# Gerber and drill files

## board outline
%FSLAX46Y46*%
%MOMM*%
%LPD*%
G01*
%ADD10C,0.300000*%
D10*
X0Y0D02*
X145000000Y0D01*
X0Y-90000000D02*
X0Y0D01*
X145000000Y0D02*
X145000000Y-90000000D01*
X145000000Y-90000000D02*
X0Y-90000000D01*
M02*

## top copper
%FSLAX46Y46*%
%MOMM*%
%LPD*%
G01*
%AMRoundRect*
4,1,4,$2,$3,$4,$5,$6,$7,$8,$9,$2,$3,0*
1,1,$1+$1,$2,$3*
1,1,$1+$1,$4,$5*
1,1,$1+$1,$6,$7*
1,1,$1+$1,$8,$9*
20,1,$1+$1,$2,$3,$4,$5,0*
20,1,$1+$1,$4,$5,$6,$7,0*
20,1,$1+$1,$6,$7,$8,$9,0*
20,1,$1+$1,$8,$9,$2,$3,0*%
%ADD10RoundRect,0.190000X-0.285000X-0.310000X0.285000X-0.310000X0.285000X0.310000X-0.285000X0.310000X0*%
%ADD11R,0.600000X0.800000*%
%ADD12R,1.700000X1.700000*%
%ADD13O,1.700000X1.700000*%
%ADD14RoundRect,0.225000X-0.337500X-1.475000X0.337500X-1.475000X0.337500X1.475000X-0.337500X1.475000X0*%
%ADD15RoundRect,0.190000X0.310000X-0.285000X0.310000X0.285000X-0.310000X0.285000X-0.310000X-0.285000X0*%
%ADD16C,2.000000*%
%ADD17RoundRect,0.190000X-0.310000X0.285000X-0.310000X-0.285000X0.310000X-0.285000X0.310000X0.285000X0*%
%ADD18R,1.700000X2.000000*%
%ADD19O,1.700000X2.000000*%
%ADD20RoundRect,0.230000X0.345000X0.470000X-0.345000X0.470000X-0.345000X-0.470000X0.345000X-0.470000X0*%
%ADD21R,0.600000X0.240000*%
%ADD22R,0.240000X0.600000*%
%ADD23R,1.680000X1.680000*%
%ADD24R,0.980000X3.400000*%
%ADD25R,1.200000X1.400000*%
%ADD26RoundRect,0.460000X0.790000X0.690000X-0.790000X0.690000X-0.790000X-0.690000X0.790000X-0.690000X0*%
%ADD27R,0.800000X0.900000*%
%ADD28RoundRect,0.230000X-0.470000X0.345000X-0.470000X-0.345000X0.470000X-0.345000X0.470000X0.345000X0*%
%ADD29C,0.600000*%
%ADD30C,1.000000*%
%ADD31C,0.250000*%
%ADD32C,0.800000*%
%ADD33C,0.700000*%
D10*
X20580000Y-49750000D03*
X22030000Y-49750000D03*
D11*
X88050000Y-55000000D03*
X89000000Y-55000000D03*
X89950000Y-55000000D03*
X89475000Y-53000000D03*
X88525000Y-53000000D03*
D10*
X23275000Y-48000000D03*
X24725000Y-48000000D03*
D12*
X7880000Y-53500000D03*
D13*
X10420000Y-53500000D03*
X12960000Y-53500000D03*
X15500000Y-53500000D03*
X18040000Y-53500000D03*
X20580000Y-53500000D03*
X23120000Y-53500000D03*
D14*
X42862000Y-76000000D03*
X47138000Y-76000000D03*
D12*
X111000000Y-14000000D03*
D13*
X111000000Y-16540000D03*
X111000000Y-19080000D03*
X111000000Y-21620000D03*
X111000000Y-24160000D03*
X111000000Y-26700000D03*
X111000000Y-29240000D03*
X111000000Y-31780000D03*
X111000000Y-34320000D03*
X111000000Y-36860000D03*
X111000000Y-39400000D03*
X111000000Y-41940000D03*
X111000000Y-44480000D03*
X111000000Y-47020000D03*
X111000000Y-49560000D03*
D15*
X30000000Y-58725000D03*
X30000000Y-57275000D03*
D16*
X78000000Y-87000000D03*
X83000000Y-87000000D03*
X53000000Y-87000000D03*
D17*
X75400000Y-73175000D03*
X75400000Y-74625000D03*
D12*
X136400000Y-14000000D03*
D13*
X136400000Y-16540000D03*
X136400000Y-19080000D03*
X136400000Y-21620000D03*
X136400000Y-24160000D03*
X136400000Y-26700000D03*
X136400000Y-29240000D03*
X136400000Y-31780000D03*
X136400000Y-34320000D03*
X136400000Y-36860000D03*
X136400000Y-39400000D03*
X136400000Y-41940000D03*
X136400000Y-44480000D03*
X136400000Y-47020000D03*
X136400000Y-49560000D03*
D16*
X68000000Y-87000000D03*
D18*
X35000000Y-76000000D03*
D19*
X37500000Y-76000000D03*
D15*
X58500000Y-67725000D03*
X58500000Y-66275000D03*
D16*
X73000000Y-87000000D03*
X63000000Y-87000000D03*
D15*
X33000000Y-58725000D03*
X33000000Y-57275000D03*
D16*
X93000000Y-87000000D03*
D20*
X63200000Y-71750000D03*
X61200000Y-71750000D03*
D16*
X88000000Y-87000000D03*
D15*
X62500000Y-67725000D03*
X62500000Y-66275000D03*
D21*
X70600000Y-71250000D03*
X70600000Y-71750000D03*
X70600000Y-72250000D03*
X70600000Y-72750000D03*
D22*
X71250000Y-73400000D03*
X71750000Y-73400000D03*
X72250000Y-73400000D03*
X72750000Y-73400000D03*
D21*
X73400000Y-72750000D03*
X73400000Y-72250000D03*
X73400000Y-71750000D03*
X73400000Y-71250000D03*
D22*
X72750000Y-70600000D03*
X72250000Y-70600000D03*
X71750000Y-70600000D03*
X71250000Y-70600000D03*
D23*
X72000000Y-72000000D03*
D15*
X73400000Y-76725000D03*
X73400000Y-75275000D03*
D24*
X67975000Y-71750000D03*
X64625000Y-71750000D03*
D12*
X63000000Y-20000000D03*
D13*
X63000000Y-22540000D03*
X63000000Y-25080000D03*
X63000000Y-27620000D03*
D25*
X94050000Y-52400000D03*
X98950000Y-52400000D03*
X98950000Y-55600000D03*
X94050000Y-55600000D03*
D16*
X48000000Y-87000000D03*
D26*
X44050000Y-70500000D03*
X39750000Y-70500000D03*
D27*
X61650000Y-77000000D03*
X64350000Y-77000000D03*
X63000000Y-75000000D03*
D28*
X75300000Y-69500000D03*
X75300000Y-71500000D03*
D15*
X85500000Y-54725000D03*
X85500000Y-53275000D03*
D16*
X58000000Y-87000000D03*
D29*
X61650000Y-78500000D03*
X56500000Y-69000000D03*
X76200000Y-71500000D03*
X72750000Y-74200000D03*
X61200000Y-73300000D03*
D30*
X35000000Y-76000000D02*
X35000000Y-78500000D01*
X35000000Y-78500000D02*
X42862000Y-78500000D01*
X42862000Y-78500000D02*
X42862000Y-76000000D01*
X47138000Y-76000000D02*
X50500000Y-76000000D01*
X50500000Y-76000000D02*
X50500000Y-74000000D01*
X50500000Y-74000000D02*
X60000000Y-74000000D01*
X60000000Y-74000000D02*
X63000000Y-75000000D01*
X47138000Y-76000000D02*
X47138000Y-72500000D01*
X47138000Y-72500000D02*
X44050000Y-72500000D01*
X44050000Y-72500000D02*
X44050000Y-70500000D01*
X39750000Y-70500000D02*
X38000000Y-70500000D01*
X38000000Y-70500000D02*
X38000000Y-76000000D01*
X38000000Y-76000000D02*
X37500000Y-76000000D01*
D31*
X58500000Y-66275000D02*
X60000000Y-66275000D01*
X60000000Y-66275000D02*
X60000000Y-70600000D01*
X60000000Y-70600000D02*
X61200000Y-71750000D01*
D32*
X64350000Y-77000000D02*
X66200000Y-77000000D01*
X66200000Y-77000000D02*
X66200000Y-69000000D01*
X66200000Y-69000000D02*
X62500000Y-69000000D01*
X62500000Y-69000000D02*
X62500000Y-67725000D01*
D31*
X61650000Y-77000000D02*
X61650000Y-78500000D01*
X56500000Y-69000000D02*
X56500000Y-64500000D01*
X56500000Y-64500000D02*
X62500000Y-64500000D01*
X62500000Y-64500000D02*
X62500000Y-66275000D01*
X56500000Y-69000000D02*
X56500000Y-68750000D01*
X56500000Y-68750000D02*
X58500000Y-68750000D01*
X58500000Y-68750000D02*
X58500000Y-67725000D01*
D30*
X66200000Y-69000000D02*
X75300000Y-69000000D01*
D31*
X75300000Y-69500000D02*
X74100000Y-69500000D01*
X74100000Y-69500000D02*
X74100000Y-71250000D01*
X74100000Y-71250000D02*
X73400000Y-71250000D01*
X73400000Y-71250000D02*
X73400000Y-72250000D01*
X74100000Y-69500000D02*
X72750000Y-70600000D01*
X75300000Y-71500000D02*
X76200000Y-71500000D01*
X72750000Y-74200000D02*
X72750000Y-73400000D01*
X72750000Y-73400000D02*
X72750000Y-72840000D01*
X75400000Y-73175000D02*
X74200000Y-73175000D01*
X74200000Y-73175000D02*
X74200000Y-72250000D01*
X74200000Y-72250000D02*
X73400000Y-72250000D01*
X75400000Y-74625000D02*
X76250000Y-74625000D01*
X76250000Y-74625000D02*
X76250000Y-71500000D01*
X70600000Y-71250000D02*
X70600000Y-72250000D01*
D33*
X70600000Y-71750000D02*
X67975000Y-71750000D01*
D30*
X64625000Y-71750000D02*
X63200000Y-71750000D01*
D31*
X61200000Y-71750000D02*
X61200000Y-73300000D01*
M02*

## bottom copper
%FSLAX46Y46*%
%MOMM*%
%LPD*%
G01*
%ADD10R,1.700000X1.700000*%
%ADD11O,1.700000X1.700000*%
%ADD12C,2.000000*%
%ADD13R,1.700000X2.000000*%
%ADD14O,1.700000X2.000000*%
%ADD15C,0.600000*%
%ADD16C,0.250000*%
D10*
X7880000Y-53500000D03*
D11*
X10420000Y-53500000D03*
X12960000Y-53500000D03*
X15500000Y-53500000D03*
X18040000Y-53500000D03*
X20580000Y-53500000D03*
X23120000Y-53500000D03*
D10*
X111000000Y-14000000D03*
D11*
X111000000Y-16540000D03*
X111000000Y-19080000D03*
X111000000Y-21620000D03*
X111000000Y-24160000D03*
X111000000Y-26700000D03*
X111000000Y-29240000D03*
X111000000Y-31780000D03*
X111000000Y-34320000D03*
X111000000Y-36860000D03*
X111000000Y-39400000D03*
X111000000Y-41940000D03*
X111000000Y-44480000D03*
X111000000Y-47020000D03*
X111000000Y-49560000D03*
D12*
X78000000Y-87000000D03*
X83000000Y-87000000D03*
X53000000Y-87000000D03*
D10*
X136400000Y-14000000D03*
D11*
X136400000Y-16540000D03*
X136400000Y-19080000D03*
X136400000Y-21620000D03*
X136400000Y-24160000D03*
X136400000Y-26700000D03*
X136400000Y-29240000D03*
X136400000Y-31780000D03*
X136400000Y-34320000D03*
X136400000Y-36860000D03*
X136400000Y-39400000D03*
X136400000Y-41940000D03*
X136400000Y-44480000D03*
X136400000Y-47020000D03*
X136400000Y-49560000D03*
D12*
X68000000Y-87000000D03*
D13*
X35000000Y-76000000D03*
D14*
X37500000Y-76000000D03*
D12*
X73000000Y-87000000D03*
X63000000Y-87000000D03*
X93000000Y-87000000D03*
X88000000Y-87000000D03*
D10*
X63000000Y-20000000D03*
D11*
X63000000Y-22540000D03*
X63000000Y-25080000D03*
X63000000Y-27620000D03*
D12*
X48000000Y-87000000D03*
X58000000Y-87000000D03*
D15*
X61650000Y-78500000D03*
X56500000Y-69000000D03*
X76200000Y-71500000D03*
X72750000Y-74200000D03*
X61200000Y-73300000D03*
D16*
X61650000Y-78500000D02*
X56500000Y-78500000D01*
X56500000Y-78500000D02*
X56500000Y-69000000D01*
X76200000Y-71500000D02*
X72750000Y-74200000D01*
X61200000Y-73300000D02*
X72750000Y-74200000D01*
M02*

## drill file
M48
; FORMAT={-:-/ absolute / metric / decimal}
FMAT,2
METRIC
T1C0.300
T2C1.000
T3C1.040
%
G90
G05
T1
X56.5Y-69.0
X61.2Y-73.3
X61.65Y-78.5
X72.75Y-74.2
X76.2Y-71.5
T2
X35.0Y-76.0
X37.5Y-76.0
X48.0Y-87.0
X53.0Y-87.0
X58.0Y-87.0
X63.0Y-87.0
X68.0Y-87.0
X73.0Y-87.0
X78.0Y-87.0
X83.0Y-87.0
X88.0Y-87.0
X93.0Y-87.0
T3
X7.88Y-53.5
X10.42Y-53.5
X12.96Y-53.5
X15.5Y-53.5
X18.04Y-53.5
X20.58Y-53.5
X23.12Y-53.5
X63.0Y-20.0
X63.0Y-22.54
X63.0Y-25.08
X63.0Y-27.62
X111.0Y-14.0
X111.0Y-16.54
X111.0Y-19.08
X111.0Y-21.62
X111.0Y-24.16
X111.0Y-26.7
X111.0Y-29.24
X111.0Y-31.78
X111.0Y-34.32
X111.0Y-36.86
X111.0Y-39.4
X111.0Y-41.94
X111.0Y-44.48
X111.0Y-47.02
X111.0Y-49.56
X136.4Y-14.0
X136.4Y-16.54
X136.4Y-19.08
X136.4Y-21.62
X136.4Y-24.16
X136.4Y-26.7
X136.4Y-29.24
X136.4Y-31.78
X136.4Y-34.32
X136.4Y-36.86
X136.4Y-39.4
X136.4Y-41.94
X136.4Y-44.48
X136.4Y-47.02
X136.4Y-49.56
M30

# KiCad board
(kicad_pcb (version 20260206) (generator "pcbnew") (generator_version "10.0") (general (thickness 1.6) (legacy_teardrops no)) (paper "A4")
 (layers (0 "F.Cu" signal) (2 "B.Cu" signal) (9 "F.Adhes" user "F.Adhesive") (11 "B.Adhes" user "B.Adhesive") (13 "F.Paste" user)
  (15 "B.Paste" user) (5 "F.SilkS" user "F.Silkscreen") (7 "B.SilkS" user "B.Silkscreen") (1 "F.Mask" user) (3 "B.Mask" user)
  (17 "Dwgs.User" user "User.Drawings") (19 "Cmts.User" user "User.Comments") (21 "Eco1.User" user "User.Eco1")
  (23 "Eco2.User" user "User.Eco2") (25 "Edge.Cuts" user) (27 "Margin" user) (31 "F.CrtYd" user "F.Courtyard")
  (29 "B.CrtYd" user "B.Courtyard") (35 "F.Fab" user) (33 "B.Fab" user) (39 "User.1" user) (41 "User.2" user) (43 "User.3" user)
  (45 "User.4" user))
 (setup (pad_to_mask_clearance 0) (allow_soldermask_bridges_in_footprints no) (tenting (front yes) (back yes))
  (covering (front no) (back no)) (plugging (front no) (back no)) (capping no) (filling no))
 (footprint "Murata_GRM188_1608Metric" (layer "F.Cu") (at 21.305 49.75)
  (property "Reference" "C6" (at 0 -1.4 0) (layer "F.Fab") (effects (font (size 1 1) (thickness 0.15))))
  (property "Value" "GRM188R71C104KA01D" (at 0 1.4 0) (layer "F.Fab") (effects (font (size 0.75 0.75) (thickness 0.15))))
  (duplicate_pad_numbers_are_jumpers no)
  (pad "1" smd roundrect (at -0.725 0) (size 0.95 1) (layers "F.Cu" "F.Mask" "F.Paste") (roundrect_rratio 0.2) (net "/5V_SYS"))
  (pad "2" smd roundrect (at 0.725 0) (size 0.95 1) (layers "F.Cu" "F.Mask" "F.Paste") (roundrect_rratio 0.2) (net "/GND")))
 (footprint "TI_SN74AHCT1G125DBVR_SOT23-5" (layer "F.Cu") (at 89 54)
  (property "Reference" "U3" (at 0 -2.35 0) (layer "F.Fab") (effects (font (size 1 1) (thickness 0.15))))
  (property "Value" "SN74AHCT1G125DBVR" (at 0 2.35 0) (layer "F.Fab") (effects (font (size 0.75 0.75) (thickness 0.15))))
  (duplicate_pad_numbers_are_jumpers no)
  (pad "1" smd rect (at -0.95 1) (size 0.6 0.8) (layers "F.Cu" "F.Mask" "F.Paste") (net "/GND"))
  (pad "2" smd rect (at 0 1) (size 0.6 0.8) (layers "F.Cu" "F.Mask" "F.Paste") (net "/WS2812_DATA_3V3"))
  (pad "3" smd rect (at 0.95 1) (size 0.6 0.8) (layers "F.Cu" "F.Mask" "F.Paste") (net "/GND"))
  (pad "4" smd rect (at 0.475 -1) (size 0.6 0.8) (layers "F.Cu" "F.Mask" "F.Paste") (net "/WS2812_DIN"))
  (pad "5" smd rect (at -0.475 -1) (size 0.6 0.8) (layers "F.Cu" "F.Mask" "F.Paste") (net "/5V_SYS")))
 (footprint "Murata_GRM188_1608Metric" (layer "F.Cu") (at 24 48)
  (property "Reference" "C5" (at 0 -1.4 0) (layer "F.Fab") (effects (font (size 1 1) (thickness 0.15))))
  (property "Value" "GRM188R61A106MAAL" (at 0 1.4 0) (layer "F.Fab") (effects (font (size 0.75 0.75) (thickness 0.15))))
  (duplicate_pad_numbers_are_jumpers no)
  (pad "1" smd roundrect (at -0.725 0) (size 0.95 1) (layers "F.Cu" "F.Mask" "F.Paste") (roundrect_rratio 0.2) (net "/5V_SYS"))
  (pad "2" smd roundrect (at 0.725 0) (size 0.95 1) (layers "F.Cu" "F.Mask" "F.Paste") (roundrect_rratio 0.2) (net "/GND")))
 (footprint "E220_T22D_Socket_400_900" (layer "F.Cu") (at 5 52)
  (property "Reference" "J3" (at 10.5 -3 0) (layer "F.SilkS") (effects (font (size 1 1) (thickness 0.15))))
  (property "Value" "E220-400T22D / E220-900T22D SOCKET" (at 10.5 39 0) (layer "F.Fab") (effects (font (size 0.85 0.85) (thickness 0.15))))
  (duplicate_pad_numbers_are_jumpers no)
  (pad "1" thru_hole rect (at 2.88 1.5) (size 1.7 1.7) (drill 1.04) (layers "*.Cu" "*.Mask") (remove_unused_layers no) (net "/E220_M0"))
  (pad "2" thru_hole oval (at 5.42 1.5) (size 1.7 1.7) (drill 1.04) (layers "*.Cu" "*.Mask") (remove_unused_layers no) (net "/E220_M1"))
  (pad "3" thru_hole oval (at 7.96 1.5) (size 1.7 1.7) (drill 1.04) (layers "*.Cu" "*.Mask") (remove_unused_layers no) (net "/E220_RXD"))
  (pad "4" thru_hole oval (at 10.5 1.5) (size 1.7 1.7) (drill 1.04) (layers "*.Cu" "*.Mask") (remove_unused_layers no) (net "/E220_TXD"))
  (pad "5" thru_hole oval (at 13.04 1.5) (size 1.7 1.7) (drill 1.04) (layers "*.Cu" "*.Mask") (remove_unused_layers no) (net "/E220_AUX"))
  (pad "6" thru_hole oval (at 15.58 1.5) (size 1.7 1.7) (drill 1.04) (layers "*.Cu" "*.Mask") (remove_unused_layers no) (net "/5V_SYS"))
  (pad "7" thru_hole oval (at 18.12 1.5) (size 1.7 1.7) (drill 1.04) (layers "*.Cu" "*.Mask") (remove_unused_layers no) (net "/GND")))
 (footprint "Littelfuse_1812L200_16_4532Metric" (layer "F.Cu") (at 45 76)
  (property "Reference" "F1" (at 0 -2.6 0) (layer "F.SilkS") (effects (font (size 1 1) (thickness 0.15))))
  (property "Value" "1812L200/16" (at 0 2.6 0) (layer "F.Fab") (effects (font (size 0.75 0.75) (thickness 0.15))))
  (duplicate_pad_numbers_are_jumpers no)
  (pad "1" smd roundrect (at -2.138 0) (size 1.125 3.4) (layers "F.Cu" "F.Mask" "F.Paste") (roundrect_rratio 0.2) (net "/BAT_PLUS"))
  (pad "2" smd roundrect (at 2.138 0) (size 1.125 3.4) (layers "F.Cu" "F.Mask" "F.Paste") (roundrect_rratio 0.2) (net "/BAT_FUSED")))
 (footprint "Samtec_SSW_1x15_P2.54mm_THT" (layer "F.Cu") (at 111 14)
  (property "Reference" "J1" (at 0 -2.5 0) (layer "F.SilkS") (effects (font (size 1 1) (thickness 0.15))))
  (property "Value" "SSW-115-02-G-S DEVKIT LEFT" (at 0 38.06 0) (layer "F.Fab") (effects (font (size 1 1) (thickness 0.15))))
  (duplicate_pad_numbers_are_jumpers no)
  (pad "1" thru_hole rect (at 0 0) (size 1.7 1.7) (drill 1.04) (layers "*.Cu" "*.Mask") (remove_unused_layers no) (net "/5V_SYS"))
  (pad "2" thru_hole oval (at 0 2.54) (size 1.7 1.7) (drill 1.04) (layers "*.Cu" "*.Mask") (remove_unused_layers no) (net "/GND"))
  (pad "3" thru_hole oval (at 0 5.08) (size 1.7 1.7) (drill 1.04) (layers "*.Cu" "*.Mask") (remove_unused_layers no))
  (pad "4" thru_hole oval (at 0 7.62) (size 1.7 1.7) (drill 1.04) (layers "*.Cu" "*.Mask") (remove_unused_layers no))
  (pad "5" thru_hole oval (at 0 10.16) (size 1.7 1.7) (drill 1.04) (layers "*.Cu" "*.Mask") (remove_unused_layers no))
  (pad "6" thru_hole oval (at 0 12.7) (size 1.7 1.7) (drill 1.04) (layers "*.Cu" "*.Mask") (remove_unused_layers no) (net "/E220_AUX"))
  (pad "7" thru_hole oval (at 0 15.24) (size 1.7 1.7) (drill 1.04) (layers "*.Cu" "*.Mask") (remove_unused_layers no) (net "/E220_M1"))
  (pad "8" thru_hole oval (at 0 17.78) (size 1.7 1.7) (drill 1.04) (layers "*.Cu" "*.Mask") (remove_unused_layers no) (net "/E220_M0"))
  (pad "9" thru_hole oval (at 0 20.32) (size 1.7 1.7) (drill 1.04) (layers "*.Cu" "*.Mask") (remove_unused_layers no))
  (pad "10" thru_hole oval (at 0 22.86) (size 1.7 1.7) (drill 1.04) (layers "*.Cu" "*.Mask") (remove_unused_layers no))
  (pad "11" thru_hole oval (at 0 25.4) (size 1.7 1.7) (drill 1.04) (layers "*.Cu" "*.Mask") (remove_unused_layers no))
  (pad "12" thru_hole oval (at 0 27.94) (size 1.7 1.7) (drill 1.04) (layers "*.Cu" "*.Mask") (remove_unused_layers no))
  (pad "13" thru_hole oval (at 0 30.48) (size 1.7 1.7) (drill 1.04) (layers "*.Cu" "*.Mask") (remove_unused_layers no))
  (pad "14" thru_hole oval (at 0 33.02) (size 1.7 1.7) (drill 1.04) (layers "*.Cu" "*.Mask") (remove_unused_layers no))
  (pad "15" thru_hole oval (at 0 35.56) (size 1.7 1.7) (drill 1.04) (layers "*.Cu" "*.Mask") (remove_unused_layers no)))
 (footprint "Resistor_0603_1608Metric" (layer "F.Cu") (at 30 58 90)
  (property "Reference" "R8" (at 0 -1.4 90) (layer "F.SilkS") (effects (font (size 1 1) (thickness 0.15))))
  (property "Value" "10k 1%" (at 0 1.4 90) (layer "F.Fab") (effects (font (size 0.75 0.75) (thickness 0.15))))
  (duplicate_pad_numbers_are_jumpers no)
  (pad "1" smd roundrect (at -0.725 0 90) (size 0.95 1) (layers "F.Cu" "F.Mask" "F.Paste") (roundrect_rratio 0.2) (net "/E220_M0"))
  (pad "2" smd roundrect (at 0.725 0 90) (size 0.95 1) (layers "F.Cu" "F.Mask" "F.Paste") (roundrect_rratio 0.2) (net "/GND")))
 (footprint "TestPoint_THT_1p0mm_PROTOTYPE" (layer "F.Cu") (at 78 87)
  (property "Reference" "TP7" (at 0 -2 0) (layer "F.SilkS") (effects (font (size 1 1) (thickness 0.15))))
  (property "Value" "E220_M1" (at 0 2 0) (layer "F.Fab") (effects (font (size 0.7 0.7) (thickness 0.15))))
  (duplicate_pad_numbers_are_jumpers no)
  (pad "1" thru_hole circle (at 0 0) (size 2 2) (drill 1) (layers "*.Cu" "*.Mask") (remove_unused_layers no) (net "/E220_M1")))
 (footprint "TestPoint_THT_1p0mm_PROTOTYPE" (layer "F.Cu") (at 83 87)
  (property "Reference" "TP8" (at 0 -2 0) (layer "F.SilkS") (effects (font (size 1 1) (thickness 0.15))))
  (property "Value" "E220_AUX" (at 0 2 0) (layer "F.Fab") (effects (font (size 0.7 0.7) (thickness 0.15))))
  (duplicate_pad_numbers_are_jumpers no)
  (pad "1" thru_hole circle (at 0 0) (size 2 2) (drill 1) (layers "*.Cu" "*.Mask") (remove_unused_layers no) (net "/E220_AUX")))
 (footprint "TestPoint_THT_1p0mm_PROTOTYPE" (layer "F.Cu") (at 53 87)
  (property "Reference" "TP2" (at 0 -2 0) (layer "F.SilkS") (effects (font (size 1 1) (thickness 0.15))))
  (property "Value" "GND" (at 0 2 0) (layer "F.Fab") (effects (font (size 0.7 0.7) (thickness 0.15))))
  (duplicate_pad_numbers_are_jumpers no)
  (pad "1" thru_hole circle (at 0 0) (size 2 2) (drill 1) (layers "*.Cu" "*.Mask") (remove_unused_layers no) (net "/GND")))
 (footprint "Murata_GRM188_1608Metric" (layer "F.Cu") (at 75.4 73.9 -90)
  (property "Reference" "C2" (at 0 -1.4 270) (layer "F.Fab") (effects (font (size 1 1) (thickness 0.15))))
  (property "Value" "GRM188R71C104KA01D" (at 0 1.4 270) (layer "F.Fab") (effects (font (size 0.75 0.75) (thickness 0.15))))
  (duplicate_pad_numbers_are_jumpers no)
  (pad "1" smd roundrect (at -0.725 0 270) (size 0.95 1) (layers "F.Cu" "F.Mask" "F.Paste") (roundrect_rratio 0.2) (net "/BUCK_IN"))
  (pad "2" smd roundrect (at 0.725 0 270) (size 0.95 1) (layers "F.Cu" "F.Mask" "F.Paste") (roundrect_rratio 0.2) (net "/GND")))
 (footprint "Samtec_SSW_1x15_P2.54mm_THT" (layer "F.Cu") (at 136.4 14)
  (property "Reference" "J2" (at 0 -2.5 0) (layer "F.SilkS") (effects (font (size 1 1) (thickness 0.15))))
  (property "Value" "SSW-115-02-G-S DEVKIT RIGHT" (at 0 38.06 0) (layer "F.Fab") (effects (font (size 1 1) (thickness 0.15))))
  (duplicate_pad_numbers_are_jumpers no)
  (pad "1" thru_hole rect (at 0 0) (size 1.7 1.7) (drill 1.04) (layers "*.Cu" "*.Mask") (remove_unused_layers no) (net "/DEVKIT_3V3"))
  (pad "2" thru_hole oval (at 0 2.54) (size 1.7 1.7) (drill 1.04) (layers "*.Cu" "*.Mask") (remove_unused_layers no) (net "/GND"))
  (pad "3" thru_hole oval (at 0 5.08) (size 1.7 1.7) (drill 1.04) (layers "*.Cu" "*.Mask") (remove_unused_layers no))
  (pad "4" thru_hole oval (at 0 7.62) (size 1.7 1.7) (drill 1.04) (layers "*.Cu" "*.Mask") (remove_unused_layers no))
  (pad "5" thru_hole oval (at 0 10.16) (size 1.7 1.7) (drill 1.04) (layers "*.Cu" "*.Mask") (remove_unused_layers no)
   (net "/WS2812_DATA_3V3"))
  (pad "6" thru_hole oval (at 0 12.7) (size 1.7 1.7) (drill 1.04) (layers "*.Cu" "*.Mask") (remove_unused_layers no) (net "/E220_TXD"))
  (pad "7" thru_hole oval (at 0 15.24) (size 1.7 1.7) (drill 1.04) (layers "*.Cu" "*.Mask") (remove_unused_layers no) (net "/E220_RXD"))
  (pad "8" thru_hole oval (at 0 17.78) (size 1.7 1.7) (drill 1.04) (layers "*.Cu" "*.Mask") (remove_unused_layers no))
  (pad "9" thru_hole oval (at 0 20.32) (size 1.7 1.7) (drill 1.04) (layers "*.Cu" "*.Mask") (remove_unused_layers no))
  (pad "10" thru_hole oval (at 0 22.86) (size 1.7 1.7) (drill 1.04) (layers "*.Cu" "*.Mask") (remove_unused_layers no))
  (pad "11" thru_hole oval (at 0 25.4) (size 1.7 1.7) (drill 1.04) (layers "*.Cu" "*.Mask") (remove_unused_layers no) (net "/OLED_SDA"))
  (pad "12" thru_hole oval (at 0 27.94) (size 1.7 1.7) (drill 1.04) (layers "*.Cu" "*.Mask") (remove_unused_layers no))
  (pad "13" thru_hole oval (at 0 30.48) (size 1.7 1.7) (drill 1.04) (layers "*.Cu" "*.Mask") (remove_unused_layers no))
  (pad "14" thru_hole oval (at 0 33.02) (size 1.7 1.7) (drill 1.04) (layers "*.Cu" "*.Mask") (remove_unused_layers no) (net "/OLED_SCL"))
  (pad "15" thru_hole oval (at 0 35.56) (size 1.7 1.7) (drill 1.04) (layers "*.Cu" "*.Mask") (remove_unused_layers no)))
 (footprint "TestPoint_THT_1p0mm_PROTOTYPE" (layer "F.Cu") (at 68 87)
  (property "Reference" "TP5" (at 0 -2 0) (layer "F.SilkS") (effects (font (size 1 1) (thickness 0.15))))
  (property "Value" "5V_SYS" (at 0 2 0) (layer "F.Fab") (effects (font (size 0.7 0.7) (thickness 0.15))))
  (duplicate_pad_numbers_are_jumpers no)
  (pad "1" thru_hole circle (at 0 0) (size 2 2) (drill 1) (layers "*.Cu" "*.Mask") (remove_unused_layers no) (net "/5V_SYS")))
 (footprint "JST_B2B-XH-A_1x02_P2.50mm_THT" (layer "F.Cu") (at 35 76)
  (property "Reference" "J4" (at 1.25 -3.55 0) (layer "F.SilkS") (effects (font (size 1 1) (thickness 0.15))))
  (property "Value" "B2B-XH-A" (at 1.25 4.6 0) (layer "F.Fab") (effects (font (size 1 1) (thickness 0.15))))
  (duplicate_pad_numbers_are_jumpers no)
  (pad "1" thru_hole rect (at 0 0) (size 1.7 2) (drill 1) (layers "*.Cu" "*.Mask") (remove_unused_layers no) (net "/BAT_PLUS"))
  (pad "2" thru_hole oval (at 2.5 0) (size 1.7 2) (drill 1) (layers "*.Cu" "*.Mask") (remove_unused_layers no) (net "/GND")))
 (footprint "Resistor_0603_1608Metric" (layer "F.Cu") (at 58.5 67 90)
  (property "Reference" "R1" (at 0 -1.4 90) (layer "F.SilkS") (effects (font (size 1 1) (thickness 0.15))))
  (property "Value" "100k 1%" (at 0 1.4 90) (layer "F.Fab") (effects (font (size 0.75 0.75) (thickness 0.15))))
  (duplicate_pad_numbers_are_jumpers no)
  (pad "1" smd roundrect (at -0.725 0 90) (size 0.95 1) (layers "F.Cu" "F.Mask" "F.Paste") (roundrect_rratio 0.2) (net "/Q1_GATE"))
  (pad "2" smd roundrect (at 0.725 0 90) (size 0.95 1) (layers "F.Cu" "F.Mask" "F.Paste") (roundrect_rratio 0.2) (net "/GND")))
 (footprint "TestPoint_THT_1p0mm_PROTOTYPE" (layer "F.Cu") (at 73 87)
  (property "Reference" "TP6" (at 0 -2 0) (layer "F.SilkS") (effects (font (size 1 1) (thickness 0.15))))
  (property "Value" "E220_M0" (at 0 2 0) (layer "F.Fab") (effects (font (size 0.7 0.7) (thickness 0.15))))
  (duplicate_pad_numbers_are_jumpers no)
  (pad "1" thru_hole circle (at 0 0) (size 2 2) (drill 1) (layers "*.Cu" "*.Mask") (remove_unused_layers no) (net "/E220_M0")))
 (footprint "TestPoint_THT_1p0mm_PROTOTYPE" (layer "F.Cu") (at 63 87)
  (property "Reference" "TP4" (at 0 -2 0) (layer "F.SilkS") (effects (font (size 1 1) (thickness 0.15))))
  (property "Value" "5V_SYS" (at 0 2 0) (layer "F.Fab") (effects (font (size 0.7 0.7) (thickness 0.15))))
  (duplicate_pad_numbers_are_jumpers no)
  (pad "1" thru_hole circle (at 0 0) (size 2 2) (drill 1) (layers "*.Cu" "*.Mask") (remove_unused_layers no) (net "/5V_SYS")))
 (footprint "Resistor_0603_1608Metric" (layer "F.Cu") (at 33 58 90)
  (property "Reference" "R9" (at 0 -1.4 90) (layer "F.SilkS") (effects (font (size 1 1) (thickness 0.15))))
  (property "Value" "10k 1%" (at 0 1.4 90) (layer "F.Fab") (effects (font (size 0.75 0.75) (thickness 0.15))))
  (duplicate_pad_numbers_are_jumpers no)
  (pad "1" smd roundrect (at -0.725 0 90) (size 0.95 1) (layers "F.Cu" "F.Mask" "F.Paste") (roundrect_rratio 0.2) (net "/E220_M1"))
  (pad "2" smd roundrect (at 0.725 0 90) (size 0.95 1) (layers "F.Cu" "F.Mask" "F.Paste") (roundrect_rratio 0.2) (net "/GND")))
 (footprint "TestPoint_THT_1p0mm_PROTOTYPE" (layer "F.Cu") (at 93 87)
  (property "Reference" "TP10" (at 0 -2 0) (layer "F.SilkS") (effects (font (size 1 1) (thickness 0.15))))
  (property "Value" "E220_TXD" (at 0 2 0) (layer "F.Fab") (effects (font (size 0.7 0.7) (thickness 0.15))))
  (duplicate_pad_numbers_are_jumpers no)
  (pad "1" thru_hole circle (at 0 0) (size 2 2) (drill 1) (layers "*.Cu" "*.Mask") (remove_unused_layers no) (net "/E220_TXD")))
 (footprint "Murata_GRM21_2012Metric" (layer "F.Cu") (at 62.2 71.75 180)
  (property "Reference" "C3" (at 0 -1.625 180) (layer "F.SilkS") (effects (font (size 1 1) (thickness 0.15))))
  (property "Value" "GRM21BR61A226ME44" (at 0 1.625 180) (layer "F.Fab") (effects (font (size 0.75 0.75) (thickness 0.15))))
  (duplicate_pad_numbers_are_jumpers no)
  (pad "1" smd roundrect (at -1 0 180) (size 1.15 1.4) (layers "F.Cu" "F.Mask" "F.Paste") (roundrect_rratio 0.2) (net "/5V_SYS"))
  (pad "2" smd roundrect (at 1 0 180) (size 1.15 1.4) (layers "F.Cu" "F.Mask" "F.Paste") (roundrect_rratio 0.2) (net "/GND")))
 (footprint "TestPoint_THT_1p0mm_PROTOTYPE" (layer "F.Cu") (at 88 87)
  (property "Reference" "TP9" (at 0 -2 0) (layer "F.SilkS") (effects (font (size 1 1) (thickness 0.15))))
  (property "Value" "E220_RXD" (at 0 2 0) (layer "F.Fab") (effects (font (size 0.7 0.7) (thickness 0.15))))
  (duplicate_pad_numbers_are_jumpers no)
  (pad "1" thru_hole circle (at 0 0) (size 2 2) (drill 1) (layers "*.Cu" "*.Mask") (remove_unused_layers no) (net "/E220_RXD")))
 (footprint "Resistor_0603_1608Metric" (layer "F.Cu") (at 62.5 67 90)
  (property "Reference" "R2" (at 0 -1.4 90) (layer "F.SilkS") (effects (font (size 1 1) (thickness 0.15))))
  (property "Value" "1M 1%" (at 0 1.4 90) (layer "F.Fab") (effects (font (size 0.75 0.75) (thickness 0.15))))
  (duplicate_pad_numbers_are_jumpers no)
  (pad "1" smd roundrect (at -0.725 0 90) (size 0.95 1) (layers "F.Cu" "F.Mask" "F.Paste") (roundrect_rratio 0.2) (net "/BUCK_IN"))
  (pad "2" smd roundrect (at 0.725 0 90) (size 0.95 1) (layers "F.Cu" "F.Mask" "F.Paste") (roundrect_rratio 0.2) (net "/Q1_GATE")))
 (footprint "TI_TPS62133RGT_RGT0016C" (layer "F.Cu") (at 72 72)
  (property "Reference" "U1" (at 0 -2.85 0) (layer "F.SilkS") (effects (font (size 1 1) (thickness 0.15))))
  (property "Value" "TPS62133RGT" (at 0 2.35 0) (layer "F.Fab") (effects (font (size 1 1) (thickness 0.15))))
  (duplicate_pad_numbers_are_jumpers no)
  (pad "" smd rect (at 0 0) (size 1.55 1.55) (layers "F.Paste"))
  (pad "1" smd rect (at -1.4 -0.75) (size 0.6 0.24) (layers "F.Cu" "F.Mask" "F.Paste") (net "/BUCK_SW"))
  (pad "2" smd rect (at -1.4 -0.25) (size 0.6 0.24) (layers "F.Cu" "F.Mask" "F.Paste") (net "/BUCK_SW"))
  (pad "3" smd rect (at -1.4 0.25) (size 0.6 0.24) (layers "F.Cu" "F.Mask" "F.Paste") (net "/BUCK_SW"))
  (pad "4" smd rect (at -1.4 0.75) (size 0.6 0.24) (layers "F.Cu" "F.Mask" "F.Paste"))
  (pad "5" smd rect (at -0.75 1.4) (size 0.24 0.6) (layers "F.Cu" "F.Mask" "F.Paste") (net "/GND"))
  (pad "6" smd rect (at -0.25 1.4) (size 0.24 0.6) (layers "F.Cu" "F.Mask" "F.Paste") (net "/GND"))
  (pad "7" smd rect (at 0.25 1.4) (size 0.24 0.6) (layers "F.Cu" "F.Mask" "F.Paste") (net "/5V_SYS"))
  (pad "8" smd rect (at 0.75 1.4) (size 0.24 0.6) (layers "F.Cu" "F.Mask" "F.Paste") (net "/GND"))
  (pad "9" smd rect (at 1.4 0.75) (size 0.6 0.24) (layers "F.Cu" "F.Mask" "F.Paste") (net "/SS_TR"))
  (pad "10" smd rect (at 1.4 0.25) (size 0.6 0.24) (layers "F.Cu" "F.Mask" "F.Paste") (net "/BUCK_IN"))
  (pad "11" smd rect (at 1.4 -0.25) (size 0.6 0.24) (layers "F.Cu" "F.Mask" "F.Paste") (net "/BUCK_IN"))
  (pad "12" smd rect (at 1.4 -0.75) (size 0.6 0.24) (layers "F.Cu" "F.Mask" "F.Paste") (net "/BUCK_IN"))
  (pad "13" smd rect (at 0.75 -1.4) (size 0.24 0.6) (layers "F.Cu" "F.Mask" "F.Paste") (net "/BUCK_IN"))
  (pad "14" smd rect (at 0.25 -1.4) (size 0.24 0.6) (layers "F.Cu" "F.Mask" "F.Paste") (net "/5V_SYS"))
  (pad "15" smd rect (at -0.25 -1.4) (size 0.24 0.6) (layers "F.Cu" "F.Mask" "F.Paste") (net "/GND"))
  (pad "16" smd rect (at -0.75 -1.4) (size 0.24 0.6) (layers "F.Cu" "F.Mask" "F.Paste") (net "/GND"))
  (pad "EP" smd rect (at 0 0) (size 1.68 1.68) (layers "F.Cu" "F.Mask") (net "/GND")))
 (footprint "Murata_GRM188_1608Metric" (layer "F.Cu") (at 73.4 76 90)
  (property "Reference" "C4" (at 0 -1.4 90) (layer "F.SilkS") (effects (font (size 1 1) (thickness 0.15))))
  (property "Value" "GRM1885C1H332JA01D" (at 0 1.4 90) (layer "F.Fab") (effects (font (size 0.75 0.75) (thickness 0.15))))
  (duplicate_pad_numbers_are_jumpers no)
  (pad "1" smd roundrect (at -0.725 0 90) (size 0.95 1) (layers "F.Cu" "F.Mask" "F.Paste") (roundrect_rratio 0.2) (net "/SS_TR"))
  (pad "2" smd roundrect (at 0.725 0 90) (size 0.95 1) (layers "F.Cu" "F.Mask" "F.Paste") (roundrect_rratio 0.2) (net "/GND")))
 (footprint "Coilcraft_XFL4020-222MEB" (layer "F.Cu") (at 66.3 71.75 180)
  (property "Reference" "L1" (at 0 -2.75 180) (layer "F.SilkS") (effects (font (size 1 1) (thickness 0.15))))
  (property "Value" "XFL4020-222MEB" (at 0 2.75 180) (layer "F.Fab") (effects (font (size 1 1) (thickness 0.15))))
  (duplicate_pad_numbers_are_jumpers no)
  (pad "1" smd rect (at -1.675 0 180) (size 0.98 3.4) (layers "F.Cu" "F.Mask" "F.Paste") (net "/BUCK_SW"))
  (pad "2" smd rect (at 1.675 0 180) (size 0.98 3.4) (layers "F.Cu" "F.Mask" "F.Paste") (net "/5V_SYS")))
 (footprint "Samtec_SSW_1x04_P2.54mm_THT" (layer "F.Cu") (at 63 20)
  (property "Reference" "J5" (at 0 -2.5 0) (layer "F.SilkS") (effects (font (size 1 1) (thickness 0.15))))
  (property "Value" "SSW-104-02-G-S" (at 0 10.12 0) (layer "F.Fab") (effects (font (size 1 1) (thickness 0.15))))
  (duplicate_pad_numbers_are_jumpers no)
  (pad "1" thru_hole rect (at 0 0) (size 1.7 1.7) (drill 1.04) (layers "*.Cu" "*.Mask") (remove_unused_layers no) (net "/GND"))
  (pad "2" thru_hole oval (at 0 2.54) (size 1.7 1.7) (drill 1.04) (layers "*.Cu" "*.Mask") (remove_unused_layers no) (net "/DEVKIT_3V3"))
  (pad "3" thru_hole oval (at 0 5.08) (size 1.7 1.7) (drill 1.04) (layers "*.Cu" "*.Mask") (remove_unused_layers no) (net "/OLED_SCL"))
  (pad "4" thru_hole oval (at 0 7.62) (size 1.7 1.7) (drill 1.04) (layers "*.Cu" "*.Mask") (remove_unused_layers no) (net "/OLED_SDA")))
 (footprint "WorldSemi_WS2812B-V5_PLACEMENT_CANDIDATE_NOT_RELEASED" (layer "F.Cu") (at 96.5 54)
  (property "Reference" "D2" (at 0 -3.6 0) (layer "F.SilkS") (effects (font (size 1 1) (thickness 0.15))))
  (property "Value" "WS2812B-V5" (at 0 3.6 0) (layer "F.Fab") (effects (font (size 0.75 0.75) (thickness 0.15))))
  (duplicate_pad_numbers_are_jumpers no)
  (pad "1" smd rect (at -2.45 -1.6) (size 1.2 1.4) (layers "F.Cu" "F.Mask" "F.Paste") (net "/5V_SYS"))
  (pad "2" smd rect (at 2.45 -1.6) (size 1.2 1.4) (layers "F.Cu" "F.Mask" "F.Paste"))
  (pad "3" smd rect (at 2.45 1.6) (size 1.2 1.4) (layers "F.Cu" "F.Mask" "F.Paste") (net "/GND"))
  (pad "4" smd rect (at -2.45 1.6) (size 1.2 1.4) (layers "F.Cu" "F.Mask" "F.Paste") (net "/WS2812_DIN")))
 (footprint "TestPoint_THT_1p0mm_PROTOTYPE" (layer "F.Cu") (at 48 87)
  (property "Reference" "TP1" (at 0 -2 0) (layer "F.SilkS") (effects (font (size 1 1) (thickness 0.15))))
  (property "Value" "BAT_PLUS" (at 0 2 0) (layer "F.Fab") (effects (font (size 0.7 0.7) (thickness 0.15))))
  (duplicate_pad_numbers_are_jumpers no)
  (pad "1" thru_hole circle (at 0 0) (size 2 2) (drill 1) (layers "*.Cu" "*.Mask") (remove_unused_layers no) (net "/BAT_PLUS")))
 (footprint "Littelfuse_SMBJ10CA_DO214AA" (layer "F.Cu") (at 41.9 70.5 180)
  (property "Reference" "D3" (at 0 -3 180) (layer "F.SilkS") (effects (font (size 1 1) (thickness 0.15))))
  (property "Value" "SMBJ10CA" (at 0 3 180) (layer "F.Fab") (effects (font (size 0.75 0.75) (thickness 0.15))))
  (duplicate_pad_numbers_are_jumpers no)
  (pad "1" smd roundrect (at -2.15 0 180) (size 2.5 2.3) (layers "F.Cu" "F.Mask" "F.Paste") (roundrect_rratio 0.2) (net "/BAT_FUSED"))
  (pad "2" smd roundrect (at 2.15 0 180) (size 2.5 2.3) (layers "F.Cu" "F.Mask" "F.Paste") (roundrect_rratio 0.2) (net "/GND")))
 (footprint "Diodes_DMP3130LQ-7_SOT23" (layer "F.Cu") (at 63 76)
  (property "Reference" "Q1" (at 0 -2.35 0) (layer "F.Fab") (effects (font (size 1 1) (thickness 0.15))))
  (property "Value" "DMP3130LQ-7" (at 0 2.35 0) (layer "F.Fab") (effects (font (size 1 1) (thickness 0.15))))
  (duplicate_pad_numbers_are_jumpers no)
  (pad "1" smd rect (at -1.35 1) (size 0.8 0.9) (layers "F.Cu" "F.Mask" "F.Paste") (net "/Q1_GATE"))
  (pad "2" smd rect (at 1.35 1) (size 0.8 0.9) (layers "F.Cu" "F.Mask" "F.Paste") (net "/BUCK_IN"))
  (pad "3" smd rect (at 0 -1) (size 0.8 0.9) (layers "F.Cu" "F.Mask" "F.Paste") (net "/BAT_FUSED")))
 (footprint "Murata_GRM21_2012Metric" (layer "F.Cu") (at 75.3 70.5 -90)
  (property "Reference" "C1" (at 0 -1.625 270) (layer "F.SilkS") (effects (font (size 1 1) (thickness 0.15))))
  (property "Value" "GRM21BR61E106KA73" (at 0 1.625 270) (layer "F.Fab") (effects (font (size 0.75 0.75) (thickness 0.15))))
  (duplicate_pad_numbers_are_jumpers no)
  (pad "1" smd roundrect (at -1 0 270) (size 1.15 1.4) (layers "F.Cu" "F.Mask" "F.Paste") (roundrect_rratio 0.2) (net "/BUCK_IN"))
  (pad "2" smd roundrect (at 1 0 270) (size 1.15 1.4) (layers "F.Cu" "F.Mask" "F.Paste") (roundrect_rratio 0.2) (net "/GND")))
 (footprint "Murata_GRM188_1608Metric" (layer "F.Cu") (at 85.5 54 90)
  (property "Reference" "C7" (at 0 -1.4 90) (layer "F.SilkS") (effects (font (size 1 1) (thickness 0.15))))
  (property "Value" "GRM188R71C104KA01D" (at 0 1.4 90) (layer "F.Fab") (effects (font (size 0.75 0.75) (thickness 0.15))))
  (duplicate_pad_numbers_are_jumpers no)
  (pad "1" smd roundrect (at -0.725 0 90) (size 0.95 1) (layers "F.Cu" "F.Mask" "F.Paste") (roundrect_rratio 0.2) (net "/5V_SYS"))
  (pad "2" smd roundrect (at 0.725 0 90) (size 0.95 1) (layers "F.Cu" "F.Mask" "F.Paste") (roundrect_rratio 0.2) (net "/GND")))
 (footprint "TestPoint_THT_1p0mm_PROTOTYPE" (layer "F.Cu") (at 58 87)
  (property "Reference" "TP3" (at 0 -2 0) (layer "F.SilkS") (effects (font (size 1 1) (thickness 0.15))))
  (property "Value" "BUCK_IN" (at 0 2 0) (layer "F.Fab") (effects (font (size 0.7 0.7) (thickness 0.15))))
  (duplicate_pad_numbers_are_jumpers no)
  (pad "1" thru_hole circle (at 0 0) (size 2 2) (drill 1) (layers "*.Cu" "*.Mask") (remove_unused_layers no) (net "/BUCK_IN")))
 (gr_line (start 0 0) (end 145 0) (stroke (width 0.3) (type default)) (layer "Edge.Cuts"))
 (gr_line (start 0 90) (end 0 0) (stroke (width 0.3) (type default)) (layer "Edge.Cuts"))
 (gr_line (start 145 0) (end 145 90) (stroke (width 0.3) (type default)) (layer "Edge.Cuts"))
 (gr_line (start 145 90) (end 0 90) (stroke (width 0.3) (type default)) (layer "Edge.Cuts"))
 (segment (start 35 76) (end 35 78.5) (width 1) (layer "F.Cu") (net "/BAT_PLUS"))
 (segment (start 35 78.5) (end 42.862 78.5) (width 1) (layer "F.Cu") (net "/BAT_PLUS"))
 (segment (start 42.862 78.5) (end 42.862 76) (width 1) (layer "F.Cu") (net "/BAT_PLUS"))
 (segment (start 47.138 76) (end 50.5 76) (width 1) (layer "F.Cu") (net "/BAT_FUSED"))
 (segment (start 50.5 76) (end 50.5 74) (width 1) (layer "F.Cu") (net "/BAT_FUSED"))
 (segment (start 50.5 74) (end 60 74) (width 1) (layer "F.Cu") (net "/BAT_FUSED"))
 (segment (start 60 74) (end 63 75) (width 1) (layer "F.Cu") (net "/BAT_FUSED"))
 (segment (start 47.138 76) (end 47.138 72.5) (width 1) (layer "F.Cu") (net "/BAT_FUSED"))
 (segment (start 47.138 72.5) (end 44.05 72.5) (width 1) (layer "F.Cu") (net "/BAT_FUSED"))
 (segment (start 44.05 72.5) (end 44.05 70.5) (width 1) (layer "F.Cu") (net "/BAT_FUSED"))
 (segment (start 39.75 70.5) (end 38 70.5) (width 1) (layer "F.Cu") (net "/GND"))
 (segment (start 38 70.5) (end 38 76) (width 1) (layer "F.Cu") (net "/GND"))
 (segment (start 38 76) (end 37.5 76) (width 1) (layer "F.Cu") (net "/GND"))
 (segment (start 58.5 66.275) (end 60 66.275) (width 0.25) (layer "F.Cu") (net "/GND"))
 (segment (start 60 66.275) (end 60 70.6) (width 0.25) (layer "F.Cu") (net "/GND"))
 (segment (start 60 70.6) (end 61.2 71.75) (width 0.25) (layer "F.Cu") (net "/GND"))
 (segment (start 64.35 77) (end 66.2 77) (width 0.8) (layer "F.Cu") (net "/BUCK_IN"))
 (segment (start 66.2 77) (end 66.2 69) (width 0.8) (layer "F.Cu") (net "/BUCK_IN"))
 (segment (start 66.2 69) (end 62.5 69) (width 0.8) (layer "F.Cu") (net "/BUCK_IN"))
 (segment (start 62.5 69) (end 62.5 67.725) (width 0.8) (layer "F.Cu") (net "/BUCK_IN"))
 (segment (start 61.65 77) (end 61.65 78.5) (width 0.25) (layer "F.Cu") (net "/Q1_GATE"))
 (via (at 61.65 78.5) (size 0.6) (drill 0.3) (layers "F.Cu" "B.Cu") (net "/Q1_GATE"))
 (segment (start 61.65 78.5) (end 56.5 78.5) (width 0.25) (layer "B.Cu") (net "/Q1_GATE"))
 (segment (start 56.5 78.5) (end 56.5 69) (width 0.25) (layer "B.Cu") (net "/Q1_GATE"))
 (via (at 56.5 69) (size 0.6) (drill 0.3) (layers "F.Cu" "B.Cu") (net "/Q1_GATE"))
 (segment (start 56.5 69) (end 56.5 64.5) (width 0.25) (layer "F.Cu") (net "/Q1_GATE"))
 (segment (start 56.5 64.5) (end 62.5 64.5) (width 0.25) (layer "F.Cu") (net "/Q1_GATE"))
 (segment (start 62.5 64.5) (end 62.5 66.275) (width 0.25) (layer "F.Cu") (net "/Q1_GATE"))
 (segment (start 56.5 69) (end 56.5 68.75) (width 0.25) (layer "F.Cu") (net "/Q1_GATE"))
 (segment (start 56.5 68.75) (end 58.5 68.75) (width 0.25) (layer "F.Cu") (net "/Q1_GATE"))
 (segment (start 58.5 68.75) (end 58.5 67.725) (width 0.25) (layer "F.Cu") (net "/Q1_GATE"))
 (segment (start 66.2 69) (end 75.3 69) (width 1) (layer "F.Cu") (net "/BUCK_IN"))
 (segment (start 75.3 69.5) (end 74.1 69.5) (width 0.25) (layer "F.Cu") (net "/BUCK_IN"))
 (segment (start 74.1 69.5) (end 74.1 71.25) (width 0.25) (layer "F.Cu") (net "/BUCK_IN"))
 (segment (start 74.1 71.25) (end 73.4 71.25) (width 0.25) (layer "F.Cu") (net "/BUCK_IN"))
 (segment (start 73.4 71.25) (end 73.4 72.25) (width 0.25) (layer "F.Cu") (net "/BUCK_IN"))
 (segment (start 74.1 69.5) (end 72.75 70.6) (width 0.25) (layer "F.Cu") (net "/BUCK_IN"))
 (segment (start 75.3 71.5) (end 76.2 71.5) (width 0.25) (layer "F.Cu") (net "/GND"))
 (via (at 76.2 71.5) (size 0.6) (drill 0.3) (layers "F.Cu" "B.Cu") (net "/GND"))
 (segment (start 76.2 71.5) (end 72.75 74.2) (width 0.25) (layer "B.Cu") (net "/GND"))
 (via (at 72.75 74.2) (size 0.6) (drill 0.3) (layers "F.Cu" "B.Cu") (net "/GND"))
 (segment (start 72.75 74.2) (end 72.75 73.4) (width 0.25) (layer "F.Cu") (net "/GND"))
 (segment (start 72.75 73.4) (end 72.75 72.84) (width 0.25) (layer "F.Cu") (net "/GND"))
 (segment (start 75.4 73.175) (end 74.2 73.175) (width 0.25) (layer "F.Cu") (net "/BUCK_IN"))
 (segment (start 74.2 73.175) (end 74.2 72.25) (width 0.25) (layer "F.Cu") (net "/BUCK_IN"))
 (segment (start 74.2 72.25) (end 73.4 72.25) (width 0.25) (layer "F.Cu") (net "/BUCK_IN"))
 (segment (start 75.4 74.625) (end 76.25 74.625) (width 0.25) (layer "F.Cu") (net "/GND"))
 (segment (start 76.25 74.625) (end 76.25 71.5) (width 0.25) (layer "F.Cu") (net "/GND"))
 (segment (start 70.6 71.25) (end 70.6 72.25) (width 0.25) (layer "F.Cu") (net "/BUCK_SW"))
 (segment (start 70.6 71.75) (end 67.975 71.75) (width 0.7) (layer "F.Cu") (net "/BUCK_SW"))
 (segment (start 64.625 71.75) (end 63.2 71.75) (width 1) (layer "F.Cu") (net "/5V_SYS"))
 (segment (start 61.2 71.75) (end 61.2 73.3) (width 0.25) (layer "F.Cu") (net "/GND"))
 (via (at 61.2 73.3) (size 0.6) (drill 0.3) (layers "F.Cu" "B.Cu") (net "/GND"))
 (segment (start 61.2 73.3) (end 72.75 74.2) (width 0.25) (layer "B.Cu") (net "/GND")))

